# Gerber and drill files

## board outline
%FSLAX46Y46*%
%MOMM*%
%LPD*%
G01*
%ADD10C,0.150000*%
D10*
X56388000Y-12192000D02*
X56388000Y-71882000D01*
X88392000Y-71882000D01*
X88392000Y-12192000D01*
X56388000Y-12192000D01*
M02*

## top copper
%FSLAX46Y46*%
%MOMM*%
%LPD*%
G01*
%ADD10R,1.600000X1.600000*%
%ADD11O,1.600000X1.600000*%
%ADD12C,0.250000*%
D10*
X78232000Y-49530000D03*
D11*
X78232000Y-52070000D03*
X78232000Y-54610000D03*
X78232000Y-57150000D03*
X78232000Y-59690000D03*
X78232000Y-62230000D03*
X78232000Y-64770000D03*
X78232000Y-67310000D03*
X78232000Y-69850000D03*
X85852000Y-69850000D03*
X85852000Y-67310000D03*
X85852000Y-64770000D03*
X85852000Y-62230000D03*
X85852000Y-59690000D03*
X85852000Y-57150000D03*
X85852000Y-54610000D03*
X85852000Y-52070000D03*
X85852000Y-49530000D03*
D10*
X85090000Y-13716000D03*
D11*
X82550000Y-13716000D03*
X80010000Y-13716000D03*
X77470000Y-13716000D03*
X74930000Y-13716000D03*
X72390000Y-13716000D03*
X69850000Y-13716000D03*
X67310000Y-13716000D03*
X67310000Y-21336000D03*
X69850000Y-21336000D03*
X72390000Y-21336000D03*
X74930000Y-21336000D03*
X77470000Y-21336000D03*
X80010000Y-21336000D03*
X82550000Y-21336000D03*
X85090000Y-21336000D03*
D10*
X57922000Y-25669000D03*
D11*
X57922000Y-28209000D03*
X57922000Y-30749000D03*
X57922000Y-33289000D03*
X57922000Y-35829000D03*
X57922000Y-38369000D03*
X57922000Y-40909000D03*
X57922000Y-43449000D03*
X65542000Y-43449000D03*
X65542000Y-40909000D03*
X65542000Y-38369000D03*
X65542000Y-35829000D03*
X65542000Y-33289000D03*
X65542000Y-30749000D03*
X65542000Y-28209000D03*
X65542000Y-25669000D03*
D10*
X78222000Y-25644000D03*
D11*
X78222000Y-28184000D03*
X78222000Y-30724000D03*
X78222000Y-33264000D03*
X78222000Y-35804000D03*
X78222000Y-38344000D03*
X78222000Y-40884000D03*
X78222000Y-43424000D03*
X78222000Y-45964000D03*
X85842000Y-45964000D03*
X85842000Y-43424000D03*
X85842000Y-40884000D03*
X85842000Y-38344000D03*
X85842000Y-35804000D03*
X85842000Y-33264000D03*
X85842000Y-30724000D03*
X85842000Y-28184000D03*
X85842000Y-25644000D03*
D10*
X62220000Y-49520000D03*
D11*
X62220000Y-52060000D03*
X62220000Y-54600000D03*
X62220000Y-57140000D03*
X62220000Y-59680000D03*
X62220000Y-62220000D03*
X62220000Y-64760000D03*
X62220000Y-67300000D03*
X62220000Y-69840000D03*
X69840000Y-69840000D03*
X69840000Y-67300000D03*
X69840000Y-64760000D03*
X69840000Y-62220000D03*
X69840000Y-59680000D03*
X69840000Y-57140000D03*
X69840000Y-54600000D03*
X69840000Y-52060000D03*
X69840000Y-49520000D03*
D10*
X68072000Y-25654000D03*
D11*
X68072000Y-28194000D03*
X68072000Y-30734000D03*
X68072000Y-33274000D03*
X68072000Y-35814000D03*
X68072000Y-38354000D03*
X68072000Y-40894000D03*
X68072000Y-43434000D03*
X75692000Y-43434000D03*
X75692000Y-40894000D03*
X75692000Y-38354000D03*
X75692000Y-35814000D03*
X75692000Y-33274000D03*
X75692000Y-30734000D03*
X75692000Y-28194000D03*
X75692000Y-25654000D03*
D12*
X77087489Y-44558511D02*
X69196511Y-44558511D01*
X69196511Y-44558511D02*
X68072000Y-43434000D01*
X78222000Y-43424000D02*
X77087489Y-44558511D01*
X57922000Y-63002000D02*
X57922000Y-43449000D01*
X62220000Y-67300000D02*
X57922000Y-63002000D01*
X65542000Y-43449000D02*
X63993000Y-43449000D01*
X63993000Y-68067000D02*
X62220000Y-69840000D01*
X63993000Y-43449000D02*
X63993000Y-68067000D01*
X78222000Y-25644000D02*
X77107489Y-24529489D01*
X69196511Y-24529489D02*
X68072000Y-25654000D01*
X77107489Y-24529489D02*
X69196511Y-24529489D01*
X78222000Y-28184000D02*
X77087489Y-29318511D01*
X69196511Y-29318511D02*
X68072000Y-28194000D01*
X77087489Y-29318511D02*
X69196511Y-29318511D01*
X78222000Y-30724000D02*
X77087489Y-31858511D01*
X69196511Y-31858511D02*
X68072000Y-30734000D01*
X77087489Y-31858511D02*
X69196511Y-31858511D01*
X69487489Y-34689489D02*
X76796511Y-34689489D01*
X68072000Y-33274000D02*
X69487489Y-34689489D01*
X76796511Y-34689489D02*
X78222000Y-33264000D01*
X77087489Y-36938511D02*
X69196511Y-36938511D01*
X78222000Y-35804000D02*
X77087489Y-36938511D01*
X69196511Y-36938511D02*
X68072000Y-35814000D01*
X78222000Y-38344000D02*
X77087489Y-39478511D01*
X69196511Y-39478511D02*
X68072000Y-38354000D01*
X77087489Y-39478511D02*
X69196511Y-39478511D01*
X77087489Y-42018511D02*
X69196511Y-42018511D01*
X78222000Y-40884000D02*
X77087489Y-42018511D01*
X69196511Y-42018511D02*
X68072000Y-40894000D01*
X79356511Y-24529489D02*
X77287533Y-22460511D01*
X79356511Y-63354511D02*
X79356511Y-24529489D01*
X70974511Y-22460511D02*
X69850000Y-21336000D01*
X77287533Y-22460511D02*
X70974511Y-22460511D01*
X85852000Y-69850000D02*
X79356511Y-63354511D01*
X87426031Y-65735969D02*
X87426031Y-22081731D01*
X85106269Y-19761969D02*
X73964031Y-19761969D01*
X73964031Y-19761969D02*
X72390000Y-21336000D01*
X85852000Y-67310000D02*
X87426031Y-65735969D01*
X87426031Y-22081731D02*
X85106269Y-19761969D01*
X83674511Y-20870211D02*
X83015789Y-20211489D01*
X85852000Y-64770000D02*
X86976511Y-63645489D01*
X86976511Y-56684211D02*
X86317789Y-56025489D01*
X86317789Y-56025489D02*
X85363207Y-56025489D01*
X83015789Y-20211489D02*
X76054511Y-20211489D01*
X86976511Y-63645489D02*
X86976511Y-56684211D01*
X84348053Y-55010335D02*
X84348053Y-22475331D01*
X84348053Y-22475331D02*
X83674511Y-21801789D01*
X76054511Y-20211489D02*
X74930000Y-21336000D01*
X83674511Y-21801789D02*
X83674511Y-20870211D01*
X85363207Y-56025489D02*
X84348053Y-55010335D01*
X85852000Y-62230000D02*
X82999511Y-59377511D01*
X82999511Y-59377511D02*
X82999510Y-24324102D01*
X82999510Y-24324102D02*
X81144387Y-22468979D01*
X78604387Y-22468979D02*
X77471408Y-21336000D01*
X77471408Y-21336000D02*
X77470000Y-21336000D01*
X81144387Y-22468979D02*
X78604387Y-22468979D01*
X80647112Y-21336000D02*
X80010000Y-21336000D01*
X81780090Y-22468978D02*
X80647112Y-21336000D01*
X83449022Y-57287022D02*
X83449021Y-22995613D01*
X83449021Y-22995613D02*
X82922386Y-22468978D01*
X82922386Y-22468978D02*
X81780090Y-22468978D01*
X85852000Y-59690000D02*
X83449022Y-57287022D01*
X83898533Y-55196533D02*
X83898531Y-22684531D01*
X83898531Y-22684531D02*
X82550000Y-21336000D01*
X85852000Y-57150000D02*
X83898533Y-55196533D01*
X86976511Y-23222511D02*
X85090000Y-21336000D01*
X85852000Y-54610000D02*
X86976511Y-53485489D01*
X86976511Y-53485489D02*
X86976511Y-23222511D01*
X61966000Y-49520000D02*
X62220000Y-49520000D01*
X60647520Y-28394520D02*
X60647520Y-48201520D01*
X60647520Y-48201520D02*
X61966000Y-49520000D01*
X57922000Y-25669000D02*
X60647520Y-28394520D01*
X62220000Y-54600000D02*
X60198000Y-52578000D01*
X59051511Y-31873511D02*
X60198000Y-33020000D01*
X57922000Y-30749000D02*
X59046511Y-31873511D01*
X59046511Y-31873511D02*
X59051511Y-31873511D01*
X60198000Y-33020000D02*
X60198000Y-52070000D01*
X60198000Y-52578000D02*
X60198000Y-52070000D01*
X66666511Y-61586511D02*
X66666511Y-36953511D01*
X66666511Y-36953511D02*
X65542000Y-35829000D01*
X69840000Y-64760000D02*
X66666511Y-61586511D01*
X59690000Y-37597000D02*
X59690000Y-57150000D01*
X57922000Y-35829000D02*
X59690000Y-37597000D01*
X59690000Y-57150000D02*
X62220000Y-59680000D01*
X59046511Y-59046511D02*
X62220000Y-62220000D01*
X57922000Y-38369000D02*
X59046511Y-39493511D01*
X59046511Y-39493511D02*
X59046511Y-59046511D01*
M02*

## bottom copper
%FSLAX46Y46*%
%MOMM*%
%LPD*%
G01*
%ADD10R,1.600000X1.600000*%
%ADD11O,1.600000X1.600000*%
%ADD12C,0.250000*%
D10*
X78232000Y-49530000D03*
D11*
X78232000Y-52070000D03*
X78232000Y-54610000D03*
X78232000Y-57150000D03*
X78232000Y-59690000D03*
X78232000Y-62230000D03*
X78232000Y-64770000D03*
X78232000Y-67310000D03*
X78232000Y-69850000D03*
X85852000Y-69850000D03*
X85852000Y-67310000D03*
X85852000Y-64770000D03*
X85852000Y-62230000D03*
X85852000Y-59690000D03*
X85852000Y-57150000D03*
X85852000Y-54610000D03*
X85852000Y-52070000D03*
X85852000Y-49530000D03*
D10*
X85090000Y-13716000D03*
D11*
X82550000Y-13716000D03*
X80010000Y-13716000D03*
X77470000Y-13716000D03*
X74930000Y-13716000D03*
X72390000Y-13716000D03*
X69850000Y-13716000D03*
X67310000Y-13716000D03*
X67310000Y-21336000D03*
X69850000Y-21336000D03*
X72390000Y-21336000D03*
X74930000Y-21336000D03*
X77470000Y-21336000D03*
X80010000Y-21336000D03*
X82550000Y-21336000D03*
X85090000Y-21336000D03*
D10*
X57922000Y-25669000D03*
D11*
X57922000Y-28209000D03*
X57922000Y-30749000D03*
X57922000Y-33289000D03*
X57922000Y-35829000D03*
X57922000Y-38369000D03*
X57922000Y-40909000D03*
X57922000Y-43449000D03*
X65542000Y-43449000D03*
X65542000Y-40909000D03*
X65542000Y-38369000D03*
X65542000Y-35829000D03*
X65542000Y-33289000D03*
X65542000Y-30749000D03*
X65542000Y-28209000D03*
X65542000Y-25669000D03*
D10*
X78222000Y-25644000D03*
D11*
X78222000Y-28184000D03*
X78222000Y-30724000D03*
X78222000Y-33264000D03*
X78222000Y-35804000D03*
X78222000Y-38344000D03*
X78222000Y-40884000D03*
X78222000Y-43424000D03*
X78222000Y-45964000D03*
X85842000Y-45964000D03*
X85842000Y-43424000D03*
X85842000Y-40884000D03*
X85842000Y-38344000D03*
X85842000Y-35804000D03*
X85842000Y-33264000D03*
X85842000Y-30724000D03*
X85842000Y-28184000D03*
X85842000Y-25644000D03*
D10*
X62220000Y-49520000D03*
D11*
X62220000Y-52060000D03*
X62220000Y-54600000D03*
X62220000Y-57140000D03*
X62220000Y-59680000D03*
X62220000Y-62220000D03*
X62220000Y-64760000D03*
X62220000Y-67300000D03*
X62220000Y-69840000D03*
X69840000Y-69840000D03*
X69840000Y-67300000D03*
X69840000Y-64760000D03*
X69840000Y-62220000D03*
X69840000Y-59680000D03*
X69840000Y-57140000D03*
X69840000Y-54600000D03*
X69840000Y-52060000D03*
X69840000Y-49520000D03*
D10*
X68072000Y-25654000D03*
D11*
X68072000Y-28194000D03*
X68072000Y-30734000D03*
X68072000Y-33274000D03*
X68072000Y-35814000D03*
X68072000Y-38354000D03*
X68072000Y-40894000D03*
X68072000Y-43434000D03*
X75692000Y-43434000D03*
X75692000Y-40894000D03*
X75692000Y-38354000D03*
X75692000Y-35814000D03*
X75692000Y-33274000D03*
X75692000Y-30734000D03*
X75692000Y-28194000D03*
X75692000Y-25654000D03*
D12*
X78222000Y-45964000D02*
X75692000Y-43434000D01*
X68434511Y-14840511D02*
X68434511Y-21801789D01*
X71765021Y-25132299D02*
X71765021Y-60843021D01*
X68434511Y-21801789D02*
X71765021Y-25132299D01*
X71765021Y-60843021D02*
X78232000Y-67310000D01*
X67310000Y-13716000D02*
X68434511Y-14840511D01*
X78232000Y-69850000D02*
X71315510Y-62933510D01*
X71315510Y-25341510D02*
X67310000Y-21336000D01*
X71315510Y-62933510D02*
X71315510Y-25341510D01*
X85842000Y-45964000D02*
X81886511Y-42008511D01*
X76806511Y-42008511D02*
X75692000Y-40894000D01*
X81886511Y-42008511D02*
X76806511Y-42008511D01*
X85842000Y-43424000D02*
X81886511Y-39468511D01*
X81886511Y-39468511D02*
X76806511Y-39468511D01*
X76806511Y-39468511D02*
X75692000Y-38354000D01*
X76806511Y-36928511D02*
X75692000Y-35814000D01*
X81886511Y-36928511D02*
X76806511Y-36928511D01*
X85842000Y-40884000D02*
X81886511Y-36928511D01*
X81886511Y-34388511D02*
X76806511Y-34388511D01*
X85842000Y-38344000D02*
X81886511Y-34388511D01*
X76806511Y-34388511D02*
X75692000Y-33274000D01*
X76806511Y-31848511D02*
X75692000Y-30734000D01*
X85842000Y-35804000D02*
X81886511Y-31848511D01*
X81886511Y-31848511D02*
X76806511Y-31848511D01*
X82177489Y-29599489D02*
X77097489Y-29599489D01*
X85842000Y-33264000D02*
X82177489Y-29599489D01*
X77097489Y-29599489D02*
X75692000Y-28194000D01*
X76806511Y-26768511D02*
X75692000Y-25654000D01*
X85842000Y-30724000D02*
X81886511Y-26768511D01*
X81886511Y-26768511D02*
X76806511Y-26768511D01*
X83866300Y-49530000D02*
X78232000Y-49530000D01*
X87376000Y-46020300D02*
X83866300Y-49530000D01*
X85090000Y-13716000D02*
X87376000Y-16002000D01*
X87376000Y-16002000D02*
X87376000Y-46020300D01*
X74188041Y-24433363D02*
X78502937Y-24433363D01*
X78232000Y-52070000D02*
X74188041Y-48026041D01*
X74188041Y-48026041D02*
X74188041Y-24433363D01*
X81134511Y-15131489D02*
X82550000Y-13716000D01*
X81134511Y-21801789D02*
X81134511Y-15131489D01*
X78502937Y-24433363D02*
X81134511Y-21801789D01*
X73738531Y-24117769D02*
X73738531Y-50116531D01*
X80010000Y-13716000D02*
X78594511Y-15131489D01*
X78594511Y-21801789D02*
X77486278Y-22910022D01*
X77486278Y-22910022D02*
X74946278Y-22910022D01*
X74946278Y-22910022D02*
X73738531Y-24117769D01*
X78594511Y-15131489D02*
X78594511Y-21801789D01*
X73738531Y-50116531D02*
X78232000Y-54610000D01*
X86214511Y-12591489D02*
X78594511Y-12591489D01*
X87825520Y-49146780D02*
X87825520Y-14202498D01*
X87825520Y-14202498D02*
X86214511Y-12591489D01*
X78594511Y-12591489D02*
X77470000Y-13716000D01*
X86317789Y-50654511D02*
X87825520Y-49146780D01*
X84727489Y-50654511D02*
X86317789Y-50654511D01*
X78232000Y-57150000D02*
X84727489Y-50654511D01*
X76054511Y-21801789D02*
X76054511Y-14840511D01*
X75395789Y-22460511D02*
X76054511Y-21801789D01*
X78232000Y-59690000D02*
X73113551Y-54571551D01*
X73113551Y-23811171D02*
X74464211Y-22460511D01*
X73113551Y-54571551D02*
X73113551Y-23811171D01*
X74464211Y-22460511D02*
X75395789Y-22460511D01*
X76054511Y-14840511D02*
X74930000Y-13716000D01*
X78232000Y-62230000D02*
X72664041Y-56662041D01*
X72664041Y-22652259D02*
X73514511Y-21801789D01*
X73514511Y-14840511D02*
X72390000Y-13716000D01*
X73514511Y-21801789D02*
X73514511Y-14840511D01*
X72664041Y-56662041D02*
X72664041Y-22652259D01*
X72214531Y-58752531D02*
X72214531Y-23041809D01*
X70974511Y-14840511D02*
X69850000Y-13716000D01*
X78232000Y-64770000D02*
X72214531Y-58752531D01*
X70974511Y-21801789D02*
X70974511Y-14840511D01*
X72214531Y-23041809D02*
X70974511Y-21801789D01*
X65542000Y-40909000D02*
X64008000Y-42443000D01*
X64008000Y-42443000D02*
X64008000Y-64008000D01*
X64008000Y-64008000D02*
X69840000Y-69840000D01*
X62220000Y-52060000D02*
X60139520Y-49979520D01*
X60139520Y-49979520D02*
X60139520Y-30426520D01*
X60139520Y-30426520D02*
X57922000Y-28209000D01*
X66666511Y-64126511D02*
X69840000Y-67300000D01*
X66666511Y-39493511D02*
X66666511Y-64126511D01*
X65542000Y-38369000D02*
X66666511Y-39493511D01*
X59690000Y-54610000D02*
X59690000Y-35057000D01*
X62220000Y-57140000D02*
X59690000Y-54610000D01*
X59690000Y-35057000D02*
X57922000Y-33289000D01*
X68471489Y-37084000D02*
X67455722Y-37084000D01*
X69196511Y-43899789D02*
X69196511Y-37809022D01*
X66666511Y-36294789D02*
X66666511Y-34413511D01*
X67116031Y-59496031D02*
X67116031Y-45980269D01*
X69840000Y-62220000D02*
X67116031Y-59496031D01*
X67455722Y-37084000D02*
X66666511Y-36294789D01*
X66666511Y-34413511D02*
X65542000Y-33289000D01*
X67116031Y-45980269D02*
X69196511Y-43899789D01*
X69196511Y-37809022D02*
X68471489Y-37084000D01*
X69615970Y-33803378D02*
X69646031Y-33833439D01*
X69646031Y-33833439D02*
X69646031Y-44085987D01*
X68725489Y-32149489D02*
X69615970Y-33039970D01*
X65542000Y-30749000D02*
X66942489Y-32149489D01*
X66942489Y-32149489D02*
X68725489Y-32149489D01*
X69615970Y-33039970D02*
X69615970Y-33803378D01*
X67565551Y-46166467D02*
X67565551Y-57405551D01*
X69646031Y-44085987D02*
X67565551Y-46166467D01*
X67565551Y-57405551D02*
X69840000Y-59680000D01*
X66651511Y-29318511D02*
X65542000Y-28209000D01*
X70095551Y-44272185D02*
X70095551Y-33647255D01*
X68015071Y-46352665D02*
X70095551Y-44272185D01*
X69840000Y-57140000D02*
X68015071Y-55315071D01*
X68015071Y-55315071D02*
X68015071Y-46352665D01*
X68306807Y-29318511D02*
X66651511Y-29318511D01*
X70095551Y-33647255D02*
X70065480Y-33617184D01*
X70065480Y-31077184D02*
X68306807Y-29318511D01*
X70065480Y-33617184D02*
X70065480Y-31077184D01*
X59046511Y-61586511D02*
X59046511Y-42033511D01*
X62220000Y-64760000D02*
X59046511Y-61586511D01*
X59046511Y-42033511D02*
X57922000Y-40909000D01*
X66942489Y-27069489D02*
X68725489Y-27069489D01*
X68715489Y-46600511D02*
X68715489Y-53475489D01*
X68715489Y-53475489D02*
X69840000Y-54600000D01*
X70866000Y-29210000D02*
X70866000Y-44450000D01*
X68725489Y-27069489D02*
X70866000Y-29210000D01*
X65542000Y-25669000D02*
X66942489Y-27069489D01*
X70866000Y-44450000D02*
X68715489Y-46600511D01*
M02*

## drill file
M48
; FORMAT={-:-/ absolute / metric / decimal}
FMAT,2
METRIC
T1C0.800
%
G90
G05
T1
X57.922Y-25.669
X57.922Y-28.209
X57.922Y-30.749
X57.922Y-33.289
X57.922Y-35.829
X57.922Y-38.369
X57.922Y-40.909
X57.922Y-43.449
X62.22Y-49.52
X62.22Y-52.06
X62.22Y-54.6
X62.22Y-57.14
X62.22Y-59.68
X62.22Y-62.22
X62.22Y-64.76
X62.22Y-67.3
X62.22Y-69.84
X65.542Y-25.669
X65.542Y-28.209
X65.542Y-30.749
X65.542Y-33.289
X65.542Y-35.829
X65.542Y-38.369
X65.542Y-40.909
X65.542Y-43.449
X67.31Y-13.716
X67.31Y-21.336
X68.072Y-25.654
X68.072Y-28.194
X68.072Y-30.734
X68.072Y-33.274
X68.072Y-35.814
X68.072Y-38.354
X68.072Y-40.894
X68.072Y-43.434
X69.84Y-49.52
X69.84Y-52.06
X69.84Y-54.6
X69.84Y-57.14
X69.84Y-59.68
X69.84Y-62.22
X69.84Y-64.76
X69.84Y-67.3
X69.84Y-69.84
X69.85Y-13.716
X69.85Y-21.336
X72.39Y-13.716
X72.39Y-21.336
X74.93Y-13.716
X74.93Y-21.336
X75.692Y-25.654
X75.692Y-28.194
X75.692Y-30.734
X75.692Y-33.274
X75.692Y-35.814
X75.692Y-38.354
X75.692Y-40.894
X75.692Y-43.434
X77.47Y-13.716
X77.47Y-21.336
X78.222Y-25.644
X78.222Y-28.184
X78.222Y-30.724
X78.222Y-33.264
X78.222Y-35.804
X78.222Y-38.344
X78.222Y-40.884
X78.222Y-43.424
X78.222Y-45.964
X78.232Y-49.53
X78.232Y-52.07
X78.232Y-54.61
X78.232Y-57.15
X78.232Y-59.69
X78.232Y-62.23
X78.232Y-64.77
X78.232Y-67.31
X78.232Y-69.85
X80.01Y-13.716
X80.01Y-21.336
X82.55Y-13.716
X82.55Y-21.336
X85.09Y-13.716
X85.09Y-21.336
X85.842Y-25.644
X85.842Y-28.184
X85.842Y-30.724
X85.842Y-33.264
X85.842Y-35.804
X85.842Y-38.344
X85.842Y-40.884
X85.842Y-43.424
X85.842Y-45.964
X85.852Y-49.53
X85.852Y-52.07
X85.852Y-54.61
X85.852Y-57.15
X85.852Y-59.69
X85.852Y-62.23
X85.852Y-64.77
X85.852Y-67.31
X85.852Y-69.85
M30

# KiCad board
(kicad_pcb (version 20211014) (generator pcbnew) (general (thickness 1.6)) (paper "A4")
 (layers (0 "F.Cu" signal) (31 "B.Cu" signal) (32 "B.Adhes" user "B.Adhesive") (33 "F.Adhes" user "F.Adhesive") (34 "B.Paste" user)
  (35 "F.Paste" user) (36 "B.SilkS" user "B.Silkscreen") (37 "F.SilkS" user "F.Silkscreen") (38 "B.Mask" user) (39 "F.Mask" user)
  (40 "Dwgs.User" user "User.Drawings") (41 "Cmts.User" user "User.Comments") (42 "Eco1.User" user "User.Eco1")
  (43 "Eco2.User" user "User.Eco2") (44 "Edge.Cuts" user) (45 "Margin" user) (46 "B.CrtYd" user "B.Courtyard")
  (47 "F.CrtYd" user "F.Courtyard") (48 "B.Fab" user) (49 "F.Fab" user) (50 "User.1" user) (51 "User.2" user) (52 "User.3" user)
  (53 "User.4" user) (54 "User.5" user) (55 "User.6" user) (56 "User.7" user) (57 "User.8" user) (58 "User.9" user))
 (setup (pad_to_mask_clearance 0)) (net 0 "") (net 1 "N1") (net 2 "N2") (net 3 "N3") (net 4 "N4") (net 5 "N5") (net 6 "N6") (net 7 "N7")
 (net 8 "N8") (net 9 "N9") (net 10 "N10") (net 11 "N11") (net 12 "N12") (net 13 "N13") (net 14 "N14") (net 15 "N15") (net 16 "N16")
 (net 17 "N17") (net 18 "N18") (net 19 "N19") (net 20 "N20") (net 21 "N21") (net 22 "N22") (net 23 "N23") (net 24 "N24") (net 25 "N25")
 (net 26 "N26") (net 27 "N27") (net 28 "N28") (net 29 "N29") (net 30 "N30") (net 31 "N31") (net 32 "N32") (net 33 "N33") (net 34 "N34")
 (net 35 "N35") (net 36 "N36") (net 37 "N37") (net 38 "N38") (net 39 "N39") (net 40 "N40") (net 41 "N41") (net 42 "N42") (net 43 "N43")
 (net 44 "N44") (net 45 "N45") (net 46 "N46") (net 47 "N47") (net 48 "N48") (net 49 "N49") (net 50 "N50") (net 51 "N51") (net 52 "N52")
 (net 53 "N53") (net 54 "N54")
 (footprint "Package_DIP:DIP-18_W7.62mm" (layer "F.Cu") (at 78.232 49.53)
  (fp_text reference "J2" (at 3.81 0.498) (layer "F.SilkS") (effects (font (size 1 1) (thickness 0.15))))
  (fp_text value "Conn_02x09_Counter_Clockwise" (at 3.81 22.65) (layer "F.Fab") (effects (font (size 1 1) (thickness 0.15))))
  (pad "1" thru_hole rect locked (at 0 0) (size 1.6 1.6) (drill 0.8) (layers *.Cu *.Mask) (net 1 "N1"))
  (pad "2" thru_hole oval locked (at 0 2.54) (size 1.6 1.6) (drill 0.8) (layers *.Cu *.Mask) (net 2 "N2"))
  (pad "3" thru_hole oval locked (at 0 5.08) (size 1.6 1.6) (drill 0.8) (layers *.Cu *.Mask) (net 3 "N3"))
  (pad "4" thru_hole oval locked (at 0 7.62) (size 1.6 1.6) (drill 0.8) (layers *.Cu *.Mask) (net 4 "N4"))
  (pad "5" thru_hole oval locked (at 0 10.16) (size 1.6 1.6) (drill 0.8) (layers *.Cu *.Mask) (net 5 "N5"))
  (pad "6" thru_hole oval locked (at 0 12.7) (size 1.6 1.6) (drill 0.8) (layers *.Cu *.Mask) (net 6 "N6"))
  (pad "7" thru_hole oval locked (at 0 15.24) (size 1.6 1.6) (drill 0.8) (layers *.Cu *.Mask) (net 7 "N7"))
  (pad "8" thru_hole oval locked (at 0 17.78) (size 1.6 1.6) (drill 0.8) (layers *.Cu *.Mask) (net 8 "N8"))
  (pad "9" thru_hole oval locked (at 0 20.32) (size 1.6 1.6) (drill 0.8) (layers *.Cu *.Mask) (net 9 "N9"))
  (pad "10" thru_hole oval locked (at 7.62 20.32) (size 1.6 1.6) (drill 0.8) (layers *.Cu *.Mask) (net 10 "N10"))
  (pad "11" thru_hole oval locked (at 7.62 17.78) (size 1.6 1.6) (drill 0.8) (layers *.Cu *.Mask) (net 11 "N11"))
  (pad "12" thru_hole oval locked (at 7.62 15.24) (size 1.6 1.6) (drill 0.8) (layers *.Cu *.Mask) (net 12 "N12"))
  (pad "13" thru_hole oval locked (at 7.62 12.7) (size 1.6 1.6) (drill 0.8) (layers *.Cu *.Mask) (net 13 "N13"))
  (pad "14" thru_hole oval locked (at 7.62 10.16) (size 1.6 1.6) (drill 0.8) (layers *.Cu *.Mask) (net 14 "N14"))
  (pad "15" thru_hole oval locked (at 7.62 7.62) (size 1.6 1.6) (drill 0.8) (layers *.Cu *.Mask) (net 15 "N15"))
  (pad "16" thru_hole oval locked (at 7.62 5.08) (size 1.6 1.6) (drill 0.8) (layers *.Cu *.Mask) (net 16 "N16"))
  (pad "17" thru_hole oval locked (at 7.62 2.54) (size 1.6 1.6) (drill 0.8) (layers *.Cu *.Mask) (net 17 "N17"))
  (pad "18" thru_hole oval locked (at 7.62 0) (size 1.6 1.6) (drill 0.8) (layers *.Cu *.Mask) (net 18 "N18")))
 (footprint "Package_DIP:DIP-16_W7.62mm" (layer "F.Cu") (at 85.09 13.716 -90)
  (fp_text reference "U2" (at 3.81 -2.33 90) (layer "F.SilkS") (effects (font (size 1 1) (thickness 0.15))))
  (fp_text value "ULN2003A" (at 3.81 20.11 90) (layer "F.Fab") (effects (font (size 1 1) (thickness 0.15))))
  (pad "1" thru_hole rect locked (at 0 0 270) (size 1.6 1.6) (drill 0.8) (layers *.Cu *.Mask) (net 1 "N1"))
  (pad "2" thru_hole oval locked (at 0 2.54 270) (size 1.6 1.6) (drill 0.8) (layers *.Cu *.Mask) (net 2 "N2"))
  (pad "3" thru_hole oval locked (at 0 5.08 270) (size 1.6 1.6) (drill 0.8) (layers *.Cu *.Mask) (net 3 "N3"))
  (pad "4" thru_hole oval locked (at 0 7.62 270) (size 1.6 1.6) (drill 0.8) (layers *.Cu *.Mask) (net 4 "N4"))
  (pad "5" thru_hole oval locked (at 0 10.16 270) (size 1.6 1.6) (drill 0.8) (layers *.Cu *.Mask) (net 5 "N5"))
  (pad "6" thru_hole oval locked (at 0 12.7 270) (size 1.6 1.6) (drill 0.8) (layers *.Cu *.Mask) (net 6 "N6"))
  (pad "7" thru_hole oval locked (at 0 15.24 270) (size 1.6 1.6) (drill 0.8) (layers *.Cu *.Mask) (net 7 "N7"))
  (pad "8" thru_hole oval locked (at 0 17.78 270) (size 1.6 1.6) (drill 0.8) (layers *.Cu *.Mask) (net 8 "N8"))
  (pad "9" thru_hole oval locked (at 7.62 17.78 270) (size 1.6 1.6) (drill 0.8) (layers *.Cu *.Mask) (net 9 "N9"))
  (pad "10" thru_hole oval locked (at 7.62 15.24 270) (size 1.6 1.6) (drill 0.8) (layers *.Cu *.Mask) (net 10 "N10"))
  (pad "11" thru_hole oval locked (at 7.62 12.7 270) (size 1.6 1.6) (drill 0.8) (layers *.Cu *.Mask) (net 11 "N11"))
  (pad "12" thru_hole oval locked (at 7.62 10.16 270) (size 1.6 1.6) (drill 0.8) (layers *.Cu *.Mask) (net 12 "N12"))
  (pad "13" thru_hole oval locked (at 7.62 7.62 270) (size 1.6 1.6) (drill 0.8) (layers *.Cu *.Mask) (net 13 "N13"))
  (pad "14" thru_hole oval locked (at 7.62 5.08 270) (size 1.6 1.6) (drill 0.8) (layers *.Cu *.Mask) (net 14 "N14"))
  (pad "15" thru_hole oval locked (at 7.62 2.54 270) (size 1.6 1.6) (drill 0.8) (layers *.Cu *.Mask) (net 15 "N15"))
  (pad "16" thru_hole oval locked (at 7.62 0 270) (size 1.6 1.6) (drill 0.8) (layers *.Cu *.Mask) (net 16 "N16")))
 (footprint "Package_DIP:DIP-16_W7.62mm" (layer "F.Cu") (at 57.922 25.669)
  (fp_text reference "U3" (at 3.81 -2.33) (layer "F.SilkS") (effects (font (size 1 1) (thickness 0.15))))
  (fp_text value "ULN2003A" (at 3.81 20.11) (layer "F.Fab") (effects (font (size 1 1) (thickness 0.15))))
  (pad "1" thru_hole rect locked (at 0 0) (size 1.6 1.6) (drill 0.8) (layers *.Cu *.Mask) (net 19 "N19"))
  (pad "2" thru_hole oval locked (at 0 2.54) (size 1.6 1.6) (drill 0.8) (layers *.Cu *.Mask) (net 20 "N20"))
  (pad "3" thru_hole oval locked (at 0 5.08) (size 1.6 1.6) (drill 0.8) (layers *.Cu *.Mask) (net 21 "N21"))
  (pad "4" thru_hole oval locked (at 0 7.62) (size 1.6 1.6) (drill 0.8) (layers *.Cu *.Mask) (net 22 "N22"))
  (pad "5" thru_hole oval locked (at 0 10.16) (size 1.6 1.6) (drill 0.8) (layers *.Cu *.Mask) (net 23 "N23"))
  (pad "6" thru_hole oval locked (at 0 12.7) (size 1.6 1.6) (drill 0.8) (layers *.Cu *.Mask) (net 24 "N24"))
  (pad "7" thru_hole oval locked (at 0 15.24) (size 1.6 1.6) (drill 0.8) (layers *.Cu *.Mask) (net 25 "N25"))
  (pad "8" thru_hole oval locked (at 0 17.78) (size 1.6 1.6) (drill 0.8) (layers *.Cu *.Mask) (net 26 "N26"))
  (pad "9" thru_hole oval locked (at 7.62 17.78) (size 1.6 1.6) (drill 0.8) (layers *.Cu *.Mask) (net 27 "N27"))
  (pad "10" thru_hole oval locked (at 7.62 15.24) (size 1.6 1.6) (drill 0.8) (layers *.Cu *.Mask) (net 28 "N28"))
  (pad "11" thru_hole oval locked (at 7.62 12.7) (size 1.6 1.6) (drill 0.8) (layers *.Cu *.Mask) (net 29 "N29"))
  (pad "12" thru_hole oval locked (at 7.62 10.16) (size 1.6 1.6) (drill 0.8) (layers *.Cu *.Mask) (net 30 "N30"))
  (pad "13" thru_hole oval locked (at 7.62 7.62) (size 1.6 1.6) (drill 0.8) (layers *.Cu *.Mask) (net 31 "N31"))
  (pad "14" thru_hole oval locked (at 7.62 5.08) (size 1.6 1.6) (drill 0.8) (layers *.Cu *.Mask) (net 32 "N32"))
  (pad "15" thru_hole oval locked (at 7.62 2.54) (size 1.6 1.6) (drill 0.8) (layers *.Cu *.Mask) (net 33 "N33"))
  (pad "16" thru_hole oval locked (at 7.62 0) (size 1.6 1.6) (drill 0.8) (layers *.Cu *.Mask) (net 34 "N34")))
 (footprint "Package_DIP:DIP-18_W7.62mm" (layer "F.Cu") (at 78.222 25.644)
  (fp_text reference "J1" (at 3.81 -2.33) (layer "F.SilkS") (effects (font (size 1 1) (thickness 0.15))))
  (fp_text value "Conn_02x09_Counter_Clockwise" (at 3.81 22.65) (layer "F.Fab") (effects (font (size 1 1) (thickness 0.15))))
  (pad "1" thru_hole rect locked (at 0 0) (size 1.6 1.6) (drill 0.8) (layers *.Cu *.Mask) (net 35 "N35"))
  (pad "2" thru_hole oval locked (at 0 2.54) (size 1.6 1.6) (drill 0.8) (layers *.Cu *.Mask) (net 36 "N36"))
  (pad "3" thru_hole oval locked (at 0 5.08) (size 1.6 1.6) (drill 0.8) (layers *.Cu *.Mask) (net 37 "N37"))
  (pad "4" thru_hole oval locked (at 0 7.62) (size 1.6 1.6) (drill 0.8) (layers *.Cu *.Mask) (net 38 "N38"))
  (pad "5" thru_hole oval locked (at 0 10.16) (size 1.6 1.6) (drill 0.8) (layers *.Cu *.Mask) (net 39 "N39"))
  (pad "6" thru_hole oval locked (at 0 12.7) (size 1.6 1.6) (drill 0.8) (layers *.Cu *.Mask) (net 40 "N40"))
  (pad "7" thru_hole oval locked (at 0 15.24) (size 1.6 1.6) (drill 0.8) (layers *.Cu *.Mask) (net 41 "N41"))
  (pad "8" thru_hole oval locked (at 0 17.78) (size 1.6 1.6) (drill 0.8) (layers *.Cu *.Mask) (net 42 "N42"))
  (pad "9" thru_hole oval locked (at 0 20.32) (size 1.6 1.6) (drill 0.8) (layers *.Cu *.Mask) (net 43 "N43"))
  (pad "10" thru_hole oval locked (at 7.62 20.32) (size 1.6 1.6) (drill 0.8) (layers *.Cu *.Mask) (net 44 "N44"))
  (pad "11" thru_hole oval locked (at 7.62 17.78) (size 1.6 1.6) (drill 0.8) (layers *.Cu *.Mask) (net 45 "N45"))
  (pad "12" thru_hole oval locked (at 7.62 15.24) (size 1.6 1.6) (drill 0.8) (layers *.Cu *.Mask) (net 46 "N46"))
  (pad "13" thru_hole oval locked (at 7.62 12.7) (size 1.6 1.6) (drill 0.8) (layers *.Cu *.Mask) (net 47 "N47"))
  (pad "14" thru_hole oval locked (at 7.62 10.16) (size 1.6 1.6) (drill 0.8) (layers *.Cu *.Mask) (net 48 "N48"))
  (pad "15" thru_hole oval locked (at 7.62 7.62) (size 1.6 1.6) (drill 0.8) (layers *.Cu *.Mask) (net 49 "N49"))
  (pad "16" thru_hole oval locked (at 7.62 5.08) (size 1.6 1.6) (drill 0.8) (layers *.Cu *.Mask) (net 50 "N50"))
  (pad "17" thru_hole oval locked (at 7.62 2.54) (size 1.6 1.6) (drill 0.8) (layers *.Cu *.Mask) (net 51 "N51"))
  (pad "18" thru_hole oval locked (at 7.62 0) (size 1.6 1.6) (drill 0.8) (layers *.Cu *.Mask) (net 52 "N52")))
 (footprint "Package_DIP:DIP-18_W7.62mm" (layer "F.Cu") (at 62.22 49.52)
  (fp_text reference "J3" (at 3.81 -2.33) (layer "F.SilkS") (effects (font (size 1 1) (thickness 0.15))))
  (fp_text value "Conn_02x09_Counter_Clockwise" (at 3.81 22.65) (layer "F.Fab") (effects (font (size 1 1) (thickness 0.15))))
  (pad "1" thru_hole rect locked (at 0 0) (size 1.6 1.6) (drill 0.8) (layers *.Cu *.Mask) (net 19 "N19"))
  (pad "2" thru_hole oval locked (at 0 2.54) (size 1.6 1.6) (drill 0.8) (layers *.Cu *.Mask) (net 20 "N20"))
  (pad "3" thru_hole oval locked (at 0 5.08) (size 1.6 1.6) (drill 0.8) (layers *.Cu *.Mask) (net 21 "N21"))
  (pad "4" thru_hole oval locked (at 0 7.62) (size 1.6 1.6) (drill 0.8) (layers *.Cu *.Mask) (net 22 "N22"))
  (pad "5" thru_hole oval locked (at 0 10.16) (size 1.6 1.6) (drill 0.8) (layers *.Cu *.Mask) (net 23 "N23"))
  (pad "6" thru_hole oval locked (at 0 12.7) (size 1.6 1.6) (drill 0.8) (layers *.Cu *.Mask) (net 24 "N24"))
  (pad "7" thru_hole oval locked (at 0 15.24) (size 1.6 1.6) (drill 0.8) (layers *.Cu *.Mask) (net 25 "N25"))
  (pad "8" thru_hole oval locked (at 0 17.78) (size 1.6 1.6) (drill 0.8) (layers *.Cu *.Mask) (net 26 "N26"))
  (pad "9" thru_hole oval locked (at 0 20.32) (size 1.6 1.6) (drill 0.8) (layers *.Cu *.Mask) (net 27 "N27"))
  (pad "10" thru_hole oval locked (at 7.62 20.32) (size 1.6 1.6) (drill 0.8) (layers *.Cu *.Mask) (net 28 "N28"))
  (pad "11" thru_hole oval locked (at 7.62 17.78) (size 1.6 1.6) (drill 0.8) (layers *.Cu *.Mask) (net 29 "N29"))
  (pad "12" thru_hole oval locked (at 7.62 15.24) (size 1.6 1.6) (drill 0.8) (layers *.Cu *.Mask) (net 30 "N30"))
  (pad "13" thru_hole oval locked (at 7.62 12.7) (size 1.6 1.6) (drill 0.8) (layers *.Cu *.Mask) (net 31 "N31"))
  (pad "14" thru_hole oval locked (at 7.62 10.16) (size 1.6 1.6) (drill 0.8) (layers *.Cu *.Mask) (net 32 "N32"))
  (pad "15" thru_hole oval locked (at 7.62 7.62) (size 1.6 1.6) (drill 0.8) (layers *.Cu *.Mask) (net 33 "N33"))
  (pad "16" thru_hole oval locked (at 7.62 5.08) (size 1.6 1.6) (drill 0.8) (layers *.Cu *.Mask) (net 34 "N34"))
  (pad "17" thru_hole oval locked (at 7.62 2.54) (size 1.6 1.6) (drill 0.8) (layers *.Cu *.Mask) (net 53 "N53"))
  (pad "18" thru_hole oval locked (at 7.62 0) (size 1.6 1.6) (drill 0.8) (layers *.Cu *.Mask) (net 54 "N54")))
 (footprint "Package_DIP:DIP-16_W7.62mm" (layer "F.Cu") (at 68.072 25.654)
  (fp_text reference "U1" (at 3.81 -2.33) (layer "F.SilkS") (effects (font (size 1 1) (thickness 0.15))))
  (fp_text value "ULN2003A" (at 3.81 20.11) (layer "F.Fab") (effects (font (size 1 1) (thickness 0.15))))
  (pad "1" thru_hole rect locked (at 0 0) (size 1.6 1.6) (drill 0.8) (layers *.Cu *.Mask) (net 35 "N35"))
  (pad "2" thru_hole oval locked (at 0 2.54) (size 1.6 1.6) (drill 0.8) (layers *.Cu *.Mask) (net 36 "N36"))
  (pad "3" thru_hole oval locked (at 0 5.08) (size 1.6 1.6) (drill 0.8) (layers *.Cu *.Mask) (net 37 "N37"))
  (pad "4" thru_hole oval locked (at 0 7.62) (size 1.6 1.6) (drill 0.8) (layers *.Cu *.Mask) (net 38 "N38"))
  (pad "5" thru_hole oval locked (at 0 10.16) (size 1.6 1.6) (drill 0.8) (layers *.Cu *.Mask) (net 39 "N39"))
  (pad "6" thru_hole oval locked (at 0 12.7) (size 1.6 1.6) (drill 0.8) (layers *.Cu *.Mask) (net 40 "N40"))
  (pad "7" thru_hole oval locked (at 0 15.24) (size 1.6 1.6) (drill 0.8) (layers *.Cu *.Mask) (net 41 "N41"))
  (pad "8" thru_hole oval locked (at 0 17.78) (size 1.6 1.6) (drill 0.8) (layers *.Cu *.Mask) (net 42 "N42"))
  (pad "9" thru_hole oval locked (at 7.62 17.78) (size 1.6 1.6) (drill 0.8) (layers *.Cu *.Mask) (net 43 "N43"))
  (pad "10" thru_hole oval locked (at 7.62 15.24) (size 1.6 1.6) (drill 0.8) (layers *.Cu *.Mask) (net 44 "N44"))
  (pad "11" thru_hole oval locked (at 7.62 12.7) (size 1.6 1.6) (drill 0.8) (layers *.Cu *.Mask) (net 45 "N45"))
  (pad "12" thru_hole oval locked (at 7.62 10.16) (size 1.6 1.6) (drill 0.8) (layers *.Cu *.Mask) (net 46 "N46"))
  (pad "13" thru_hole oval locked (at 7.62 7.62) (size 1.6 1.6) (drill 0.8) (layers *.Cu *.Mask) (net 47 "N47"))
  (pad "14" thru_hole oval locked (at 7.62 5.08) (size 1.6 1.6) (drill 0.8) (layers *.Cu *.Mask) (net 48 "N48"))
  (pad "15" thru_hole oval locked (at 7.62 2.54) (size 1.6 1.6) (drill 0.8) (layers *.Cu *.Mask) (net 49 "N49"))
  (pad "16" thru_hole oval locked (at 7.62 0) (size 1.6 1.6) (drill 0.8) (layers *.Cu *.Mask) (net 50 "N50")))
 (gr_poly (pts (xy 56.388 12.192) (xy 56.388 71.882) (xy 88.392 71.882) (xy 88.392 12.192)) (layer "Edge.Cuts") (width 0.15) (fill none))
 (segment (start 77.087489 44.558511) (end 69.196511 44.558511) (width 0.25) (layer "F.Cu") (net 42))
 (segment (start 69.196511 44.558511) (end 68.072 43.434) (width 0.25) (layer "F.Cu") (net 42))
 (segment (start 78.222 43.424) (end 77.087489 44.558511) (width 0.25) (layer "F.Cu") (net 42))
 (segment (start 78.222 45.964) (end 75.692 43.434) (width 0.25) (layer "B.Cu") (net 43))
 (segment (start 68.434511 14.840511) (end 68.434511 21.801789) (width 0.25) (layer "B.Cu") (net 8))
 (segment (start 71.765021 25.132299) (end 71.765021 60.843021) (width 0.25) (layer "B.Cu") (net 8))
 (segment (start 68.434511 21.801789) (end 71.765021 25.132299) (width 0.25) (layer "B.Cu") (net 8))
 (segment (start 71.765021 60.843021) (end 78.232 67.31) (width 0.25) (layer "B.Cu") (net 8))
 (segment (start 67.31 13.716) (end 68.434511 14.840511) (width 0.25) (layer "B.Cu") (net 8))
 (segment (start 78.232 69.85) (end 71.31551 62.93351) (width 0.25) (layer "B.Cu") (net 9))
 (segment (start 71.31551 25.34151) (end 67.31 21.336) (width 0.25) (layer "B.Cu") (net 9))
 (segment (start 71.31551 62.93351) (end 71.31551 25.34151) (width 0.25) (layer "B.Cu") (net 9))
 (segment (start 57.922 63.002) (end 57.922 43.449) (width 0.25) (layer "F.Cu") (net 26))
 (segment (start 62.22 67.3) (end 57.922 63.002) (width 0.25) (layer "F.Cu") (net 26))
 (segment (start 65.542 43.449) (end 63.993 43.449) (width 0.25) (layer "F.Cu") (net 27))
 (segment (start 63.993 68.067) (end 62.22 69.84) (width 0.25) (layer "F.Cu") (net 27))
 (segment (start 63.993 43.449) (end 63.993 68.067) (width 0.25) (layer "F.Cu") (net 27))
 (segment (start 78.222 25.644) (end 77.107489 24.529489) (width 0.25) (layer "F.Cu") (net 35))
 (segment (start 69.196511 24.529489) (end 68.072 25.654) (width 0.25) (layer "F.Cu") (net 35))
 (segment (start 77.107489 24.529489) (end 69.196511 24.529489) (width 0.25) (layer "F.Cu") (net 35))
 (segment (start 85.842 45.964) (end 81.886511 42.008511) (width 0.25) (layer "B.Cu") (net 44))
 (segment (start 76.806511 42.008511) (end 75.692 40.894) (width 0.25) (layer "B.Cu") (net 44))
 (segment (start 81.886511 42.008511) (end 76.806511 42.008511) (width 0.25) (layer "B.Cu") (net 44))
 (segment (start 78.222 28.184) (end 77.087489 29.318511) (width 0.25) (layer "F.Cu") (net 36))
 (segment (start 69.196511 29.318511) (end 68.072 28.194) (width 0.25) (layer "F.Cu") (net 36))
 (segment (start 77.087489 29.318511) (end 69.196511 29.318511) (width 0.25) (layer "F.Cu") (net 36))
 (segment (start 85.842 43.424) (end 81.886511 39.468511) (width 0.25) (layer "B.Cu") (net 45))
 (segment (start 81.886511 39.468511) (end 76.806511 39.468511) (width 0.25) (layer "B.Cu") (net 45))
 (segment (start 76.806511 39.468511) (end 75.692 38.354) (width 0.25) (layer "B.Cu") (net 45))
 (segment (start 78.222 30.724) (end 77.087489 31.858511) (width 0.25) (layer "F.Cu") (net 37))
 (segment (start 69.196511 31.858511) (end 68.072 30.734) (width 0.25) (layer "F.Cu") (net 37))
 (segment (start 77.087489 31.858511) (end 69.196511 31.858511) (width 0.25) (layer "F.Cu") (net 37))
 (segment (start 76.806511 36.928511) (end 75.692 35.814) (width 0.25) (layer "B.Cu") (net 46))
 (segment (start 81.886511 36.928511) (end 76.806511 36.928511) (width 0.25) (layer "B.Cu") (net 46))
 (segment (start 85.842 40.884) (end 81.886511 36.928511) (width 0.25) (layer "B.Cu") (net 46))
 (segment (start 69.487489 34.689489) (end 76.796511 34.689489) (width 0.25) (layer "F.Cu") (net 38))
 (segment (start 68.072 33.274) (end 69.487489 34.689489) (width 0.25) (layer "F.Cu") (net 38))
 (segment (start 76.796511 34.689489) (end 78.222 33.264) (width 0.25) (layer "F.Cu") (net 38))
 (segment (start 81.886511 34.388511) (end 76.806511 34.388511) (width 0.25) (layer "B.Cu") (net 47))
 (segment (start 85.842 38.344) (end 81.886511 34.388511) (width 0.25) (layer "B.Cu") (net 47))
 (segment (start 76.806511 34.388511) (end 75.692 33.274) (width 0.25) (layer "B.Cu") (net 47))
 (segment (start 77.087489 36.938511) (end 69.196511 36.938511) (width 0.25) (layer "F.Cu") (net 39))
 (segment (start 78.222 35.804) (end 77.087489 36.938511) (width 0.25) (layer "F.Cu") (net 39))
 (segment (start 69.196511 36.938511) (end 68.072 35.814) (width 0.25) (layer "F.Cu") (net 39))
 (segment (start 76.806511 31.848511) (end 75.692 30.734) (width 0.25) (layer "B.Cu") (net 48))
 (segment (start 85.842 35.804) (end 81.886511 31.848511) (width 0.25) (layer "B.Cu") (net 48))
 (segment (start 81.886511 31.848511) (end 76.806511 31.848511) (width 0.25) (layer "B.Cu") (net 48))
 (segment (start 78.222 38.344) (end 77.087489 39.478511) (width 0.25) (layer "F.Cu") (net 40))
 (segment (start 69.196511 39.478511) (end 68.072 38.354) (width 0.25) (layer "F.Cu") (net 40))
 (segment (start 77.087489 39.478511) (end 69.196511 39.478511) (width 0.25) (layer "F.Cu") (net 40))
 (segment (start 82.177489 29.599489) (end 77.097489 29.599489) (width 0.25) (layer "B.Cu") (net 49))
 (segment (start 85.842 33.264) (end 82.177489 29.599489) (width 0.25) (layer "B.Cu") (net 49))
 (segment (start 77.097489 29.599489) (end 75.692 28.194) (width 0.25) (layer "B.Cu") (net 49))
 (segment (start 77.087489 42.018511) (end 69.196511 42.018511) (width 0.25) (layer "F.Cu") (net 41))
 (segment (start 78.222 40.884) (end 77.087489 42.018511) (width 0.25) (layer "F.Cu") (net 41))
 (segment (start 69.196511 42.018511) (end 68.072 40.894) (width 0.25) (layer "F.Cu") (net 41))
 (segment (start 76.806511 26.768511) (end 75.692 25.654) (width 0.25) (layer "B.Cu") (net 50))
 (segment (start 85.842 30.724) (end 81.886511 26.768511) (width 0.25) (layer "B.Cu") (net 50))
 (segment (start 81.886511 26.768511) (end 76.806511 26.768511) (width 0.25) (layer "B.Cu") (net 50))
 (segment (start 83.8663 49.53) (end 78.232 49.53) (width 0.25) (layer "B.Cu") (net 1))
 (segment (start 87.376 46.0203) (end 83.8663 49.53) (width 0.25) (layer "B.Cu") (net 1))
 (segment (start 85.09 13.716) (end 87.376 16.002) (width 0.25) (layer "B.Cu") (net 1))
 (segment (start 87.376 16.002) (end 87.376 46.0203) (width 0.25) (layer "B.Cu") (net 1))
 (segment (start 79.356511 24.529489) (end 77.287533 22.460511) (width 0.25) (layer "F.Cu") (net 10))
 (segment (start 79.356511 63.354511) (end 79.356511 24.529489) (width 0.25) (layer "F.Cu") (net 10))
 (segment (start 70.974511 22.460511) (end 69.85 21.336) (width 0.25) (layer "F.Cu") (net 10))
 (segment (start 77.287533 22.460511) (end 70.974511 22.460511) (width 0.25) (layer "F.Cu") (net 10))
 (segment (start 85.852 69.85) (end 79.356511 63.354511) (width 0.25) (layer "F.Cu") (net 10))
 (segment (start 74.188041 24.433363) (end 78.502937 24.433363) (width 0.25) (layer "B.Cu") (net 2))
 (segment (start 78.232 52.07) (end 74.188041 48.026041) (width 0.25) (layer "B.Cu") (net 2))
 (segment (start 74.188041 48.026041) (end 74.188041 24.433363) (width 0.25) (layer "B.Cu") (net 2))
 (segment (start 81.134511 15.131489) (end 82.55 13.716) (width 0.25) (layer "B.Cu") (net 2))
 (segment (start 81.134511 21.801789) (end 81.134511 15.131489) (width 0.25) (layer "B.Cu") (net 2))
 (segment (start 78.502937 24.433363) (end 81.134511 21.801789) (width 0.25) (layer "B.Cu") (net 2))
 (segment (start 87.426031 65.735969) (end 87.426031 22.081731) (width 0.25) (layer "F.Cu") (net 11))
 (segment (start 85.106269 19.761969) (end 73.964031 19.761969) (width 0.25) (layer "F.Cu") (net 11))
 (segment (start 73.964031 19.761969) (end 72.39 21.336) (width 0.25) (layer "F.Cu") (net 11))
 (segment (start 85.852 67.31) (end 87.426031 65.735969) (width 0.25) (layer "F.Cu") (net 11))
 (segment (start 87.426031 22.081731) (end 85.106269 19.761969) (width 0.25) (layer "F.Cu") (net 11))
 (segment (start 73.738531 24.117769) (end 73.738531 50.116531) (width 0.25) (layer "B.Cu") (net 3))
 (segment (start 80.01 13.716) (end 78.594511 15.131489) (width 0.25) (layer "B.Cu") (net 3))
 (segment (start 78.594511 21.801789) (end 77.486278 22.910022) (width 0.25) (layer "B.Cu") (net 3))
 (segment (start 77.486278 22.910022) (end 74.946278 22.910022) (width 0.25) (layer "B.Cu") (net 3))
 (segment (start 74.946278 22.910022) (end 73.738531 24.117769) (width 0.25) (layer "B.Cu") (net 3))
 (segment (start 78.594511 15.131489) (end 78.594511 21.801789) (width 0.25) (layer "B.Cu") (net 3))
 (segment (start 73.738531 50.116531) (end 78.232 54.61) (width 0.25) (layer "B.Cu") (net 3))
 (segment (start 83.674511 20.870211) (end 83.015789 20.211489) (width 0.25) (layer "F.Cu") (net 12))
 (segment (start 85.852 64.77) (end 86.976511 63.645489) (width 0.25) (layer "F.Cu") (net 12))
 (segment (start 86.976511 56.684211) (end 86.317789 56.025489) (width 0.25) (layer "F.Cu") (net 12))
 (segment (start 86.317789 56.025489) (end 85.363207 56.025489) (width 0.25) (layer "F.Cu") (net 12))
 (segment (start 83.015789 20.211489) (end 76.054511 20.211489) (width 0.25) (layer "F.Cu") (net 12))
 (segment (start 86.976511 63.645489) (end 86.976511 56.684211) (width 0.25) (layer "F.Cu") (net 12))
 (segment (start 84.348053 55.010335) (end 84.348053 22.475331) (width 0.25) (layer "F.Cu") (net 12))
 (segment (start 84.348053 22.475331) (end 83.674511 21.801789) (width 0.25) (layer "F.Cu") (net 12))
 (segment (start 76.054511 20.211489) (end 74.93 21.336) (width 0.25) (layer "F.Cu") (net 12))
 (segment (start 83.674511 21.801789) (end 83.674511 20.870211) (width 0.25) (layer "F.Cu") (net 12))
 (segment (start 85.363207 56.025489) (end 84.348053 55.010335) (width 0.25) (layer "F.Cu") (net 12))
 (segment (start 86.214511 12.591489) (end 78.594511 12.591489) (width 0.25) (layer "B.Cu") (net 4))
 (segment (start 87.82552 49.14678) (end 87.82552 14.202498) (width 0.25) (layer "B.Cu") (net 4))
 (segment (start 87.82552 14.202498) (end 86.214511 12.591489) (width 0.25) (layer "B.Cu") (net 4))
 (segment (start 78.594511 12.591489) (end 77.47 13.716) (width 0.25) (layer "B.Cu") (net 4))
 (segment (start 86.317789 50.654511) (end 87.82552 49.14678) (width 0.25) (layer "B.Cu") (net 4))
 (segment (start 84.727489 50.654511) (end 86.317789 50.654511) (width 0.25) (layer "B.Cu") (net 4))
 (segment (start 78.232 57.15) (end 84.727489 50.654511) (width 0.25) (layer "B.Cu") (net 4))
 (segment (start 85.852 62.23) (end 82.999511 59.377511) (width 0.25) (layer "F.Cu") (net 13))
 (segment (start 82.999511 59.377511) (end 82.99951 24.324102) (width 0.25) (layer "F.Cu") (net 13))
 (segment (start 82.99951 24.324102) (end 81.144387 22.468979) (width 0.25) (layer "F.Cu") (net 13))
 (segment (start 78.604387 22.468979) (end 77.471408 21.336) (width 0.25) (layer "F.Cu") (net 13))
 (segment (start 77.471408 21.336) (end 77.47 21.336) (width 0.25) (layer "F.Cu") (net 13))
 (segment (start 81.144387 22.468979) (end 78.604387 22.468979) (width 0.25) (layer "F.Cu") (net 13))
 (segment (start 76.054511 21.801789) (end 76.054511 14.840511) (width 0.25) (layer "B.Cu") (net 5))
 (segment (start 75.395789 22.460511) (end 76.054511 21.801789) (width 0.25) (layer "B.Cu") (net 5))
 (segment (start 78.232 59.69) (end 73.113551 54.571551) (width 0.25) (layer "B.Cu") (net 5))
 (segment (start 73.113551 23.811171) (end 74.464211 22.460511) (width 0.25) (layer "B.Cu") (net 5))
 (segment (start 73.113551 54.571551) (end 73.113551 23.811171) (width 0.25) (layer "B.Cu") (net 5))
 (segment (start 74.464211 22.460511) (end 75.395789 22.460511) (width 0.25) (layer "B.Cu") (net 5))
 (segment (start 76.054511 14.840511) (end 74.93 13.716) (width 0.25) (layer "B.Cu") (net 5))
 (segment (start 80.647112 21.336) (end 80.01 21.336) (width 0.25) (layer "F.Cu") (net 14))
 (segment (start 81.78009 22.468978) (end 80.647112 21.336) (width 0.25) (layer "F.Cu") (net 14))
 (segment (start 83.449022 57.287022) (end 83.449021 22.995613) (width 0.25) (layer "F.Cu") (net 14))
 (segment (start 83.449021 22.995613) (end 82.922386 22.468978) (width 0.25) (layer "F.Cu") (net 14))
 (segment (start 82.922386 22.468978) (end 81.78009 22.468978) (width 0.25) (layer "F.Cu") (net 14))
 (segment (start 85.852 59.69) (end 83.449022 57.287022) (width 0.25) (layer "F.Cu") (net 14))
 (segment (start 78.232 62.23) (end 72.664041 56.662041) (width 0.25) (layer "B.Cu") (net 6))
 (segment (start 72.664041 22.652259) (end 73.514511 21.801789) (width 0.25) (layer "B.Cu") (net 6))
 (segment (start 73.514511 14.840511) (end 72.39 13.716) (width 0.25) (layer "B.Cu") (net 6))
 (segment (start 73.514511 21.801789) (end 73.514511 14.840511) (width 0.25) (layer "B.Cu") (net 6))
 (segment (start 72.664041 56.662041) (end 72.664041 22.652259) (width 0.25) (layer "B.Cu") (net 6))
 (segment (start 83.898533 55.196533) (end 83.898531 22.684531) (width 0.25) (layer "F.Cu") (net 15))
 (segment (start 83.898531 22.684531) (end 82.55 21.336) (width 0.25) (layer "F.Cu") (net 15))
 (segment (start 85.852 57.15) (end 83.898533 55.196533) (width 0.25) (layer "F.Cu") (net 15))
 (segment (start 72.214531 58.752531) (end 72.214531 23.041809) (width 0.25) (layer "B.Cu") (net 7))
 (segment (start 70.974511 14.840511) (end 69.85 13.716) (width 0.25) (layer "B.Cu") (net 7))
 (segment (start 78.232 64.77) (end 72.214531 58.752531) (width 0.25) (layer "B.Cu") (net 7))
 (segment (start 70.974511 21.801789) (end 70.974511 14.840511) (width 0.25) (layer "B.Cu") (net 7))
 (segment (start 72.214531 23.041809) (end 70.974511 21.801789) (width 0.25) (layer "B.Cu") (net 7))
 (segment (start 86.976511 23.222511) (end 85.09 21.336) (width 0.25) (layer "F.Cu") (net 16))
 (segment (start 85.852 54.61) (end 86.976511 53.485489) (width 0.25) (layer "F.Cu") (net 16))
 (segment (start 86.976511 53.485489) (end 86.976511 23.222511) (width 0.25) (layer "F.Cu") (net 16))
 (segment (start 61.966 49.52) (end 62.22 49.52) (width 0.25) (layer "F.Cu") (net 19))
 (segment (start 60.64752 28.39452) (end 60.64752 48.20152) (width 0.25) (layer "F.Cu") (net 19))
 (segment (start 60.64752 48.20152) (end 61.966 49.52) (width 0.25) (layer "F.Cu") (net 19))
 (segment (start 57.922 25.669) (end 60.64752 28.39452) (width 0.25) (layer "F.Cu") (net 19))
 (segment (start 65.542 40.909) (end 64.008 42.443) (width 0.25) (layer "B.Cu") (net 28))
 (segment (start 64.008 42.443) (end 64.008 64.008) (width 0.25) (layer "B.Cu") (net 28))
 (segment (start 64.008 64.008) (end 69.84 69.84) (width 0.25) (layer "B.Cu") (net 28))
 (segment (start 62.22 52.06) (end 60.13952 49.97952) (width 0.25) (layer "B.Cu") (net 20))
 (segment (start 60.13952 49.97952) (end 60.13952 30.42652) (width 0.25) (layer "B.Cu") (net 20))
 (segment (start 60.13952 30.42652) (end 57.922 28.209) (width 0.25) (layer "B.Cu") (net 20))
 (segment (start 66.666511 64.126511) (end 69.84 67.3) (width 0.25) (layer "B.Cu") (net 29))
 (segment (start 66.666511 39.493511) (end 66.666511 64.126511) (width 0.25) (layer "B.Cu") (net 29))
 (segment (start 65.542 38.369) (end 66.666511 39.493511) (width 0.25) (layer "B.Cu") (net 29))
 (segment (start 62.22 54.6) (end 60.198 52.578) (width 0.25) (layer "F.Cu") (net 21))
 (segment (start 59.051511 31.873511) (end 60.198 33.02) (width 0.25) (layer "F.Cu") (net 21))
 (segment (start 57.922 30.749) (end 59.046511 31.873511) (width 0.25) (layer "F.Cu") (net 21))
 (segment (start 59.046511 31.873511) (end 59.051511 31.873511) (width 0.25) (layer "F.Cu") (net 21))
 (segment (start 60.198 33.02) (end 60.198 52.07) (width 0.25) (layer "F.Cu") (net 21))
 (segment (start 60.198 52.578) (end 60.198 52.07) (width 0.25) (layer "F.Cu") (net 21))
 (segment (start 66.666511 61.586511) (end 66.666511 36.953511) (width 0.25) (layer "F.Cu") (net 30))
 (segment (start 66.666511 36.953511) (end 65.542 35.829) (width 0.25) (layer "F.Cu") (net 30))
 (segment (start 69.84 64.76) (end 66.666511 61.586511) (width 0.25) (layer "F.Cu") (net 30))
 (segment (start 59.69 54.61) (end 59.69 35.057) (width 0.25) (layer "B.Cu") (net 22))
 (segment (start 62.22 57.14) (end 59.69 54.61) (width 0.25) (layer "B.Cu") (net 22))
 (segment (start 59.69 35.057) (end 57.922 33.289) (width 0.25) (layer "B.Cu") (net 22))
 (segment (start 68.471489 37.084) (end 67.455722 37.084) (width 0.25) (layer "B.Cu") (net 31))
 (segment (start 69.196511 43.899789) (end 69.196511 37.809022) (width 0.25) (layer "B.Cu") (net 31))
 (segment (start 66.666511 36.294789) (end 66.666511 34.413511) (width 0.25) (layer "B.Cu") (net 31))
 (segment (start 67.116031 59.496031) (end 67.116031 45.980269) (width 0.25) (layer "B.Cu") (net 31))
 (segment (start 69.84 62.22) (end 67.116031 59.496031) (width 0.25) (layer "B.Cu") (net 31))
 (segment (start 67.455722 37.084) (end 66.666511 36.294789) (width 0.25) (layer "B.Cu") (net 31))
 (segment (start 66.666511 34.413511) (end 65.542 33.289) (width 0.25) (layer "B.Cu") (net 31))
 (segment (start 67.116031 45.980269) (end 69.196511 43.899789) (width 0.25) (layer "B.Cu") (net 31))
 (segment (start 69.196511 37.809022) (end 68.471489 37.084) (width 0.25) (layer "B.Cu") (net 31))
 (segment (start 59.69 37.597) (end 59.69 57.15) (width 0.25) (layer "F.Cu") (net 23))
 (segment (start 57.922 35.829) (end 59.69 37.597) (width 0.25) (layer "F.Cu") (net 23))
 (segment (start 59.69 57.15) (end 62.22 59.68) (width 0.25) (layer "F.Cu") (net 23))
 (segment (start 69.61597 33.803378) (end 69.646031 33.833439) (width 0.25) (layer "B.Cu") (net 32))
 (segment (start 69.646031 33.833439) (end 69.646031 44.085987) (width 0.25) (layer "B.Cu") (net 32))
 (segment (start 68.725489 32.149489) (end 69.61597 33.03997) (width 0.25) (layer "B.Cu") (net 32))
 (segment (start 65.542 30.749) (end 66.942489 32.149489) (width 0.25) (layer "B.Cu") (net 32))
 (segment (start 66.942489 32.149489) (end 68.725489 32.149489) (width 0.25) (layer "B.Cu") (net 32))
 (segment (start 69.61597 33.03997) (end 69.61597 33.803378) (width 0.25) (layer "B.Cu") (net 32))
 (segment (start 67.565551 46.166467) (end 67.565551 57.405551) (width 0.25) (layer "B.Cu") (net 32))
 (segment (start 69.646031 44.085987) (end 67.565551 46.166467) (width 0.25) (layer "B.Cu") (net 32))
 (segment (start 67.565551 57.405551) (end 69.84 59.68) (width 0.25) (layer "B.Cu") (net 32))
 (segment (start 59.046511 59.046511) (end 62.22 62.22) (width 0.25) (layer "F.Cu") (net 24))
 (segment (start 57.922 38.369) (end 59.046511 39.493511) (width 0.25) (layer "F.Cu") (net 24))
 (segment (start 59.046511 39.493511) (end 59.046511 59.046511) (width 0.25) (layer "F.Cu") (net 24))
 (segment (start 66.651511 29.318511) (end 65.542 28.209) (width 0.25) (layer "B.Cu") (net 33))
 (segment (start 70.095551 44.272185) (end 70.095551 33.647255) (width 0.25) (layer "B.Cu") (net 33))
 (segment (start 68.015071 46.352665) (end 70.095551 44.272185) (width 0.25) (layer "B.Cu") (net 33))
 (segment (start 69.84 57.14) (end 68.015071 55.315071) (width 0.25) (layer "B.Cu") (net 33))
 (segment (start 68.015071 55.315071) (end 68.015071 46.352665) (width 0.25) (layer "B.Cu") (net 33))
 (segment (start 68.306807 29.318511) (end 66.651511 29.318511) (width 0.25) (layer "B.Cu") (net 33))
 (segment (start 70.095551 33.647255) (end 70.06548 33.617184) (width 0.25) (layer "B.Cu") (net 33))
 (segment (start 70.06548 31.077184) (end 68.306807 29.318511) (width 0.25) (layer "B.Cu") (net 33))
 (segment (start 70.06548 33.617184) (end 70.06548 31.077184) (width 0.25) (layer "B.Cu") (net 33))
 (segment (start 59.046511 61.586511) (end 59.046511 42.033511) (width 0.25) (layer "B.Cu") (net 25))
 (segment (start 62.22 64.76) (end 59.046511 61.586511) (width 0.25) (layer "B.Cu") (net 25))
 (segment (start 59.046511 42.033511) (end 57.922 40.909) (width 0.25) (layer "B.Cu") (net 25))
 (segment (start 66.942489 27.069489) (end 68.725489 27.069489) (width 0.25) (layer "B.Cu") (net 34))
 (segment (start 68.715489 46.600511) (end 68.715489 53.475489) (width 0.25) (layer "B.Cu") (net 34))
 (segment (start 68.715489 53.475489) (end 69.84 54.6) (width 0.25) (layer "B.Cu") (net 34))
 (segment (start 70.866 29.21) (end 70.866 44.45) (width 0.25) (layer "B.Cu") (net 34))
 (segment (start 68.725489 27.069489) (end 70.866 29.21) (width 0.25) (layer "B.Cu") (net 34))
 (segment (start 65.542 25.669) (end 66.942489 27.069489) (width 0.25) (layer "B.Cu") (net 34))
 (segment (start 70.866 44.45) (end 68.715489 46.600511) (width 0.25) (layer "B.Cu") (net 34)))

